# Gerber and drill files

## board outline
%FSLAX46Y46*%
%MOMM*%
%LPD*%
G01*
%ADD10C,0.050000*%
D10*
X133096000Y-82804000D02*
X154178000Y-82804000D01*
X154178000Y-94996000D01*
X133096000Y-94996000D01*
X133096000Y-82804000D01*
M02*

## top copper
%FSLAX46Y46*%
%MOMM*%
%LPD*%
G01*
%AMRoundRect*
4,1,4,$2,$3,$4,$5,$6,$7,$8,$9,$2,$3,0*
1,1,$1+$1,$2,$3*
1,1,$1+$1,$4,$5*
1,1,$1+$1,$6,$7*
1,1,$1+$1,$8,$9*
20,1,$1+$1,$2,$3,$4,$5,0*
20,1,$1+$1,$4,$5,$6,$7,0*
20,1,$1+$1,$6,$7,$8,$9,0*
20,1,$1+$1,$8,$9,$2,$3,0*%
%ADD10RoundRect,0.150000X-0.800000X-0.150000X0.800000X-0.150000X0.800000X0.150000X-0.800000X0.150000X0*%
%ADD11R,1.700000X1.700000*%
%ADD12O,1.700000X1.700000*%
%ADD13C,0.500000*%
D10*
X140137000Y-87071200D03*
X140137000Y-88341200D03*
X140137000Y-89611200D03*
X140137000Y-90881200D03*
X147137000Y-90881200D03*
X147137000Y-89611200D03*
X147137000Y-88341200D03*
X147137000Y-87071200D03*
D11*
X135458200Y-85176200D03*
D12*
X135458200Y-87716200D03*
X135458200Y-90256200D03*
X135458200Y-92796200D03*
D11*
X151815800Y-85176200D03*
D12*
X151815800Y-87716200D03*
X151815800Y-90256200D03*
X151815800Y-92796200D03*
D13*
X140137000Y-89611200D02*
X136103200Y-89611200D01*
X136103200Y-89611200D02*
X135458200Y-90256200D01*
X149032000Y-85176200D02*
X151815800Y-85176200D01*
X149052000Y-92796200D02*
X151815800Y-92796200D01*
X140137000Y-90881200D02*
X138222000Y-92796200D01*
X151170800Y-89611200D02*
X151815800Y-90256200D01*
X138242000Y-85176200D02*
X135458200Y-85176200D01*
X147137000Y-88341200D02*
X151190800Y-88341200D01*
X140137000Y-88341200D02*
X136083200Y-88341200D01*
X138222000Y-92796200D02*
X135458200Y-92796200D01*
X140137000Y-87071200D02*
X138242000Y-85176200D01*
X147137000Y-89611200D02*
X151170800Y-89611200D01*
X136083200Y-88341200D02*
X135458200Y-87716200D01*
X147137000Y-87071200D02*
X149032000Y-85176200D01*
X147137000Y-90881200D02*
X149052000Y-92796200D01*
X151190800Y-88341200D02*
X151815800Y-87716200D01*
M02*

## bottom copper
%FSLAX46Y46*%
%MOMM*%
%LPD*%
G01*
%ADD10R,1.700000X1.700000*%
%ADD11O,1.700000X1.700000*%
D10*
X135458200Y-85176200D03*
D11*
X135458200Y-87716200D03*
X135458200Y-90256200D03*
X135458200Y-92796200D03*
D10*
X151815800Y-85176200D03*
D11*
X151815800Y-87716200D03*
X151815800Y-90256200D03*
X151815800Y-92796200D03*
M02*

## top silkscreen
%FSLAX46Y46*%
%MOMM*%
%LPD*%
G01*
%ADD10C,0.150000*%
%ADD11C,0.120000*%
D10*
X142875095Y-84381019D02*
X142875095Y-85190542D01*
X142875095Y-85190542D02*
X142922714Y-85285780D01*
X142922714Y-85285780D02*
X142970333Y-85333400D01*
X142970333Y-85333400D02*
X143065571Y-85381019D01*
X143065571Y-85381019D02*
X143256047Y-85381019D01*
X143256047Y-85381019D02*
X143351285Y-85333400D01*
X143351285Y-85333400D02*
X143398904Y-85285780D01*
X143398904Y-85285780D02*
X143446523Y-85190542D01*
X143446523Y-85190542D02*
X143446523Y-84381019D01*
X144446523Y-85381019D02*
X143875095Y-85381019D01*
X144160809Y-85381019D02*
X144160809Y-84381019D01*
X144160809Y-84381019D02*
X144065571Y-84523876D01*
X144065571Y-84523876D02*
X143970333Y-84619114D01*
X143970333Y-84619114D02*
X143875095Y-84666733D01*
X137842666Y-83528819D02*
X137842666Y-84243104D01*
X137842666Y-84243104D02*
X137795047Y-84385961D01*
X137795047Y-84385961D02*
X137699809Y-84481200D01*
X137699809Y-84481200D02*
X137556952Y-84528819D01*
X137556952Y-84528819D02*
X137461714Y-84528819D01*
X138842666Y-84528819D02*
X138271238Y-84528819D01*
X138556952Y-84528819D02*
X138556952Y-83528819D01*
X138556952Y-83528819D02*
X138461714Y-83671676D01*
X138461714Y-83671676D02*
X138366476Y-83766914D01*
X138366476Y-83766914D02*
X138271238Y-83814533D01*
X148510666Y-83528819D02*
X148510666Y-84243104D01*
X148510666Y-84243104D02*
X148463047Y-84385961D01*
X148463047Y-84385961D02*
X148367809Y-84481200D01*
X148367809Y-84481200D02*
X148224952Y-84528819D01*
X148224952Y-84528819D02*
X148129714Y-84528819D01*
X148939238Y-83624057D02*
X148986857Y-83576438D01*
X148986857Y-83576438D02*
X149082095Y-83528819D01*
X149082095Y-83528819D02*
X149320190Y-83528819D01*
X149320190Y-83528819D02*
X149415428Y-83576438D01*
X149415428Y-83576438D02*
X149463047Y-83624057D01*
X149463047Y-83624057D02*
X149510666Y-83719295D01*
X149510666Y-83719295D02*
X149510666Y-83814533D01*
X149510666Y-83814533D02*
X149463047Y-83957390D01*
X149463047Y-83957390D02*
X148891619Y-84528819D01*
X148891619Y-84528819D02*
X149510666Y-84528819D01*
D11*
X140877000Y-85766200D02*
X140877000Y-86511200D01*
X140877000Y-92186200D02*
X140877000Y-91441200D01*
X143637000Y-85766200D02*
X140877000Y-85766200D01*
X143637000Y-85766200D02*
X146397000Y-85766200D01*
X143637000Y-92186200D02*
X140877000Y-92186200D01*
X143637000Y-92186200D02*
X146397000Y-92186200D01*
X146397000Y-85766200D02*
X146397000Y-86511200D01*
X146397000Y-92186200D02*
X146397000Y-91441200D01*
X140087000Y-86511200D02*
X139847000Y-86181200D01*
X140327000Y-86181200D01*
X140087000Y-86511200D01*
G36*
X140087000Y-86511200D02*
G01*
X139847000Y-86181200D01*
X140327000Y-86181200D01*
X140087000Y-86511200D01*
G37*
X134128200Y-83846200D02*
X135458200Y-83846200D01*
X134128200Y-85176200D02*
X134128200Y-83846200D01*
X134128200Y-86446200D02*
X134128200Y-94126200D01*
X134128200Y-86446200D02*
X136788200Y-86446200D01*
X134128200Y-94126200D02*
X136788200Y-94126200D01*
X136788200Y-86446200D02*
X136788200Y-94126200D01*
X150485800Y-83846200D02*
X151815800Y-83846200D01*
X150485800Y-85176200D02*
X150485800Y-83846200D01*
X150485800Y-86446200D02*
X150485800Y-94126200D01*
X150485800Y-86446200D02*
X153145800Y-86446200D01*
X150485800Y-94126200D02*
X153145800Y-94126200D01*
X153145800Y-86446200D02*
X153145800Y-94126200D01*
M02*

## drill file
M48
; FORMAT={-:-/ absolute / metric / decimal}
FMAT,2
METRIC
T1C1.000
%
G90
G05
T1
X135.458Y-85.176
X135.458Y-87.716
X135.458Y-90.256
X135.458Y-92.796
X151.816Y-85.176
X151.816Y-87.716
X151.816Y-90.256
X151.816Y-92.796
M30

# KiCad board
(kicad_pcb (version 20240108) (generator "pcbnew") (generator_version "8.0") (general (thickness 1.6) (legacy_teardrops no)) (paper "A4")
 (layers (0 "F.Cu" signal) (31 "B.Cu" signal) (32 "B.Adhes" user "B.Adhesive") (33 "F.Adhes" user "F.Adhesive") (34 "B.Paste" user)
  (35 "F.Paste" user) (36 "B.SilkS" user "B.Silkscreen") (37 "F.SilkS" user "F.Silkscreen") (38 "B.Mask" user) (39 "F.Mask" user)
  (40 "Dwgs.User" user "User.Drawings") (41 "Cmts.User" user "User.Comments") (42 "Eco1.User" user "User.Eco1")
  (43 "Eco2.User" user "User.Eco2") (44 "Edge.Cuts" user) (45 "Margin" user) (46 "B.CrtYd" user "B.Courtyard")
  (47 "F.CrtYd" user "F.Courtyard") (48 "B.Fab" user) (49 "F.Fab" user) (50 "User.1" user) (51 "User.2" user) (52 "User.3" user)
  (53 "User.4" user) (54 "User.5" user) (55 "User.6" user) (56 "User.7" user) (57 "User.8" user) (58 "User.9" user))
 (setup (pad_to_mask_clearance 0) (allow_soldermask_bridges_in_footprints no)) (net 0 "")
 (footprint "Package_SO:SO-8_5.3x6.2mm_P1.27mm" (layer "F.Cu") (at 143.637 88.9762)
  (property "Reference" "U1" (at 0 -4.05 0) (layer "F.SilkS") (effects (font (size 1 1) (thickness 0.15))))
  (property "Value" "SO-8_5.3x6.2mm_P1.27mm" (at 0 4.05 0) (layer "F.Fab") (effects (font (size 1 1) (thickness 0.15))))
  (fp_line (start -2.76 -3.21) (end -2.76 -2.465) (stroke (width 0.12) (type solid)) (layer "F.SilkS"))
  (fp_line (start -2.76 3.21) (end -2.76 2.465) (stroke (width 0.12) (type solid)) (layer "F.SilkS"))
  (fp_line (start 0 -3.21) (end -2.76 -3.21) (stroke (width 0.12) (type solid)) (layer "F.SilkS"))
  (fp_line (start 0 -3.21) (end 2.76 -3.21) (stroke (width 0.12) (type solid)) (layer "F.SilkS"))
  (fp_line (start 0 3.21) (end -2.76 3.21) (stroke (width 0.12) (type solid)) (layer "F.SilkS"))
  (fp_line (start 0 3.21) (end 2.76 3.21) (stroke (width 0.12) (type solid)) (layer "F.SilkS"))
  (fp_line (start 2.76 -3.21) (end 2.76 -2.465) (stroke (width 0.12) (type solid)) (layer "F.SilkS"))
  (fp_line (start 2.76 3.21) (end 2.76 2.465) (stroke (width 0.12) (type solid)) (layer "F.SilkS"))
  (fp_poly
   (pts (xy -3.55 -2.465) (xy -3.79 -2.795) (xy -3.31 -2.795) (xy -3.55 -2.465)) (stroke (width 0.12) (type solid)) (fill solid)
   (layer "F.SilkS"))
  (pad "1" smd roundrect (at -3.5 -1.905) (size 1.9 0.6) (layers "F.Cu" "F.Paste" "F.Mask") (roundrect_rratio 0.25))
  (pad "2" smd roundrect (at -3.5 -0.635) (size 1.9 0.6) (layers "F.Cu" "F.Paste" "F.Mask") (roundrect_rratio 0.25))
  (pad "3" smd roundrect (at -3.5 0.635) (size 1.9 0.6) (layers "F.Cu" "F.Paste" "F.Mask") (roundrect_rratio 0.25))
  (pad "4" smd roundrect (at -3.5 1.905) (size 1.9 0.6) (layers "F.Cu" "F.Paste" "F.Mask") (roundrect_rratio 0.25))
  (pad "5" smd roundrect (at 3.5 1.905) (size 1.9 0.6) (layers "F.Cu" "F.Paste" "F.Mask") (roundrect_rratio 0.25))
  (pad "6" smd roundrect (at 3.5 0.635) (size 1.9 0.6) (layers "F.Cu" "F.Paste" "F.Mask") (roundrect_rratio 0.25))
  (pad "7" smd roundrect (at 3.5 -0.635) (size 1.9 0.6) (layers "F.Cu" "F.Paste" "F.Mask") (roundrect_rratio 0.25))
  (pad "8" smd roundrect (at 3.5 -1.905) (size 1.9 0.6) (layers "F.Cu" "F.Paste" "F.Mask") (roundrect_rratio 0.25)))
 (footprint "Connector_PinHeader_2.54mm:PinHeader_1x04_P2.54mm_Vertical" (layer "F.Cu") (at 135.4582 85.1762)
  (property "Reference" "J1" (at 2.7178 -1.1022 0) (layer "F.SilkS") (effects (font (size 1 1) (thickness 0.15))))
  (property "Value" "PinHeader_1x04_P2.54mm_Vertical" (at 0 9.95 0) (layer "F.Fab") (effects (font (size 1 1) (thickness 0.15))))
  (fp_line (start -1.33 -1.33) (end 0 -1.33) (stroke (width 0.12) (type solid)) (layer "F.SilkS"))
  (fp_line (start -1.33 0) (end -1.33 -1.33) (stroke (width 0.12) (type solid)) (layer "F.SilkS"))
  (fp_line (start -1.33 1.27) (end -1.33 8.95) (stroke (width 0.12) (type solid)) (layer "F.SilkS"))
  (fp_line (start -1.33 1.27) (end 1.33 1.27) (stroke (width 0.12) (type solid)) (layer "F.SilkS"))
  (fp_line (start -1.33 8.95) (end 1.33 8.95) (stroke (width 0.12) (type solid)) (layer "F.SilkS"))
  (fp_line (start 1.33 1.27) (end 1.33 8.95) (stroke (width 0.12) (type solid)) (layer "F.SilkS"))
  (pad "1" thru_hole rect (at 0 0) (size 1.7 1.7) (drill 1) (layers "*.Cu" "*.Mask") (remove_unused_layers no))
  (pad "2" thru_hole oval (at 0 2.54) (size 1.7 1.7) (drill 1) (layers "*.Cu" "*.Mask") (remove_unused_layers no))
  (pad "3" thru_hole oval (at 0 5.08) (size 1.7 1.7) (drill 1) (layers "*.Cu" "*.Mask") (remove_unused_layers no))
  (pad "4" thru_hole oval (at 0 7.62) (size 1.7 1.7) (drill 1) (layers "*.Cu" "*.Mask") (remove_unused_layers no)))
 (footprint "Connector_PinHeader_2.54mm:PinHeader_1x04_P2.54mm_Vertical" (layer "F.Cu") (at 151.8158 85.1762)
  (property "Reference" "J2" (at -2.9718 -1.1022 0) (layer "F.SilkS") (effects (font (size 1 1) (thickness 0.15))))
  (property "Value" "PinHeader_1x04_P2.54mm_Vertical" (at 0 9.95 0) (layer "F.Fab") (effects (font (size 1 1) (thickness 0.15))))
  (fp_line (start -1.33 -1.33) (end 0 -1.33) (stroke (width 0.12) (type solid)) (layer "F.SilkS"))
  (fp_line (start -1.33 0) (end -1.33 -1.33) (stroke (width 0.12) (type solid)) (layer "F.SilkS"))
  (fp_line (start -1.33 1.27) (end -1.33 8.95) (stroke (width 0.12) (type solid)) (layer "F.SilkS"))
  (fp_line (start -1.33 1.27) (end 1.33 1.27) (stroke (width 0.12) (type solid)) (layer "F.SilkS"))
  (fp_line (start -1.33 8.95) (end 1.33 8.95) (stroke (width 0.12) (type solid)) (layer "F.SilkS"))
  (fp_line (start 1.33 1.27) (end 1.33 8.95) (stroke (width 0.12) (type solid)) (layer "F.SilkS"))
  (pad "1" thru_hole rect (at 0 0) (size 1.7 1.7) (drill 1) (layers "*.Cu" "*.Mask") (remove_unused_layers no))
  (pad "2" thru_hole oval (at 0 2.54) (size 1.7 1.7) (drill 1) (layers "*.Cu" "*.Mask") (remove_unused_layers no))
  (pad "3" thru_hole oval (at 0 5.08) (size 1.7 1.7) (drill 1) (layers "*.Cu" "*.Mask") (remove_unused_layers no))
  (pad "4" thru_hole oval (at 0 7.62) (size 1.7 1.7) (drill 1) (layers "*.Cu" "*.Mask") (remove_unused_layers no)))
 (gr_rect (start 133.096 82.804) (end 154.178 94.996) (stroke (width 0.05) (type default)) (fill none) (layer "Edge.Cuts"))
 (segment (start 140.137 89.6112) (end 136.1032 89.6112) (width 0.5) (layer "F.Cu") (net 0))
 (segment (start 136.1032 89.6112) (end 135.4582 90.2562) (width 0.5) (layer "F.Cu") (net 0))
 (segment (start 149.032 85.1762) (end 151.8158 85.1762) (width 0.5) (layer "F.Cu") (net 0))
 (segment (start 149.052 92.7962) (end 151.8158 92.7962) (width 0.5) (layer "F.Cu") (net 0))
 (segment (start 140.137 90.8812) (end 138.222 92.7962) (width 0.5) (layer "F.Cu") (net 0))
 (segment (start 151.1708 89.6112) (end 151.8158 90.2562) (width 0.5) (layer "F.Cu") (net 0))
 (segment (start 138.242 85.1762) (end 135.4582 85.1762) (width 0.5) (layer "F.Cu") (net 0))
 (segment (start 147.137 88.3412) (end 151.1908 88.3412) (width 0.5) (layer "F.Cu") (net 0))
 (segment (start 140.137 88.3412) (end 136.0832 88.3412) (width 0.5) (layer "F.Cu") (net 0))
 (segment (start 138.222 92.7962) (end 135.4582 92.7962) (width 0.5) (layer "F.Cu") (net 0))
 (segment (start 140.137 87.0712) (end 138.242 85.1762) (width 0.5) (layer "F.Cu") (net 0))
 (segment (start 147.137 89.6112) (end 151.1708 89.6112) (width 0.5) (layer "F.Cu") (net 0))
 (segment (start 136.0832 88.3412) (end 135.4582 87.7162) (width 0.5) (layer "F.Cu") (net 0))
 (segment (start 147.137 87.0712) (end 149.032 85.1762) (width 0.5) (layer "F.Cu") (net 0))
 (segment (start 147.137 90.8812) (end 149.052 92.7962) (width 0.5) (layer "F.Cu") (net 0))
 (segment (start 151.1908 88.3412) (end 151.8158 87.7162) (width 0.5) (layer "F.Cu") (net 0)))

